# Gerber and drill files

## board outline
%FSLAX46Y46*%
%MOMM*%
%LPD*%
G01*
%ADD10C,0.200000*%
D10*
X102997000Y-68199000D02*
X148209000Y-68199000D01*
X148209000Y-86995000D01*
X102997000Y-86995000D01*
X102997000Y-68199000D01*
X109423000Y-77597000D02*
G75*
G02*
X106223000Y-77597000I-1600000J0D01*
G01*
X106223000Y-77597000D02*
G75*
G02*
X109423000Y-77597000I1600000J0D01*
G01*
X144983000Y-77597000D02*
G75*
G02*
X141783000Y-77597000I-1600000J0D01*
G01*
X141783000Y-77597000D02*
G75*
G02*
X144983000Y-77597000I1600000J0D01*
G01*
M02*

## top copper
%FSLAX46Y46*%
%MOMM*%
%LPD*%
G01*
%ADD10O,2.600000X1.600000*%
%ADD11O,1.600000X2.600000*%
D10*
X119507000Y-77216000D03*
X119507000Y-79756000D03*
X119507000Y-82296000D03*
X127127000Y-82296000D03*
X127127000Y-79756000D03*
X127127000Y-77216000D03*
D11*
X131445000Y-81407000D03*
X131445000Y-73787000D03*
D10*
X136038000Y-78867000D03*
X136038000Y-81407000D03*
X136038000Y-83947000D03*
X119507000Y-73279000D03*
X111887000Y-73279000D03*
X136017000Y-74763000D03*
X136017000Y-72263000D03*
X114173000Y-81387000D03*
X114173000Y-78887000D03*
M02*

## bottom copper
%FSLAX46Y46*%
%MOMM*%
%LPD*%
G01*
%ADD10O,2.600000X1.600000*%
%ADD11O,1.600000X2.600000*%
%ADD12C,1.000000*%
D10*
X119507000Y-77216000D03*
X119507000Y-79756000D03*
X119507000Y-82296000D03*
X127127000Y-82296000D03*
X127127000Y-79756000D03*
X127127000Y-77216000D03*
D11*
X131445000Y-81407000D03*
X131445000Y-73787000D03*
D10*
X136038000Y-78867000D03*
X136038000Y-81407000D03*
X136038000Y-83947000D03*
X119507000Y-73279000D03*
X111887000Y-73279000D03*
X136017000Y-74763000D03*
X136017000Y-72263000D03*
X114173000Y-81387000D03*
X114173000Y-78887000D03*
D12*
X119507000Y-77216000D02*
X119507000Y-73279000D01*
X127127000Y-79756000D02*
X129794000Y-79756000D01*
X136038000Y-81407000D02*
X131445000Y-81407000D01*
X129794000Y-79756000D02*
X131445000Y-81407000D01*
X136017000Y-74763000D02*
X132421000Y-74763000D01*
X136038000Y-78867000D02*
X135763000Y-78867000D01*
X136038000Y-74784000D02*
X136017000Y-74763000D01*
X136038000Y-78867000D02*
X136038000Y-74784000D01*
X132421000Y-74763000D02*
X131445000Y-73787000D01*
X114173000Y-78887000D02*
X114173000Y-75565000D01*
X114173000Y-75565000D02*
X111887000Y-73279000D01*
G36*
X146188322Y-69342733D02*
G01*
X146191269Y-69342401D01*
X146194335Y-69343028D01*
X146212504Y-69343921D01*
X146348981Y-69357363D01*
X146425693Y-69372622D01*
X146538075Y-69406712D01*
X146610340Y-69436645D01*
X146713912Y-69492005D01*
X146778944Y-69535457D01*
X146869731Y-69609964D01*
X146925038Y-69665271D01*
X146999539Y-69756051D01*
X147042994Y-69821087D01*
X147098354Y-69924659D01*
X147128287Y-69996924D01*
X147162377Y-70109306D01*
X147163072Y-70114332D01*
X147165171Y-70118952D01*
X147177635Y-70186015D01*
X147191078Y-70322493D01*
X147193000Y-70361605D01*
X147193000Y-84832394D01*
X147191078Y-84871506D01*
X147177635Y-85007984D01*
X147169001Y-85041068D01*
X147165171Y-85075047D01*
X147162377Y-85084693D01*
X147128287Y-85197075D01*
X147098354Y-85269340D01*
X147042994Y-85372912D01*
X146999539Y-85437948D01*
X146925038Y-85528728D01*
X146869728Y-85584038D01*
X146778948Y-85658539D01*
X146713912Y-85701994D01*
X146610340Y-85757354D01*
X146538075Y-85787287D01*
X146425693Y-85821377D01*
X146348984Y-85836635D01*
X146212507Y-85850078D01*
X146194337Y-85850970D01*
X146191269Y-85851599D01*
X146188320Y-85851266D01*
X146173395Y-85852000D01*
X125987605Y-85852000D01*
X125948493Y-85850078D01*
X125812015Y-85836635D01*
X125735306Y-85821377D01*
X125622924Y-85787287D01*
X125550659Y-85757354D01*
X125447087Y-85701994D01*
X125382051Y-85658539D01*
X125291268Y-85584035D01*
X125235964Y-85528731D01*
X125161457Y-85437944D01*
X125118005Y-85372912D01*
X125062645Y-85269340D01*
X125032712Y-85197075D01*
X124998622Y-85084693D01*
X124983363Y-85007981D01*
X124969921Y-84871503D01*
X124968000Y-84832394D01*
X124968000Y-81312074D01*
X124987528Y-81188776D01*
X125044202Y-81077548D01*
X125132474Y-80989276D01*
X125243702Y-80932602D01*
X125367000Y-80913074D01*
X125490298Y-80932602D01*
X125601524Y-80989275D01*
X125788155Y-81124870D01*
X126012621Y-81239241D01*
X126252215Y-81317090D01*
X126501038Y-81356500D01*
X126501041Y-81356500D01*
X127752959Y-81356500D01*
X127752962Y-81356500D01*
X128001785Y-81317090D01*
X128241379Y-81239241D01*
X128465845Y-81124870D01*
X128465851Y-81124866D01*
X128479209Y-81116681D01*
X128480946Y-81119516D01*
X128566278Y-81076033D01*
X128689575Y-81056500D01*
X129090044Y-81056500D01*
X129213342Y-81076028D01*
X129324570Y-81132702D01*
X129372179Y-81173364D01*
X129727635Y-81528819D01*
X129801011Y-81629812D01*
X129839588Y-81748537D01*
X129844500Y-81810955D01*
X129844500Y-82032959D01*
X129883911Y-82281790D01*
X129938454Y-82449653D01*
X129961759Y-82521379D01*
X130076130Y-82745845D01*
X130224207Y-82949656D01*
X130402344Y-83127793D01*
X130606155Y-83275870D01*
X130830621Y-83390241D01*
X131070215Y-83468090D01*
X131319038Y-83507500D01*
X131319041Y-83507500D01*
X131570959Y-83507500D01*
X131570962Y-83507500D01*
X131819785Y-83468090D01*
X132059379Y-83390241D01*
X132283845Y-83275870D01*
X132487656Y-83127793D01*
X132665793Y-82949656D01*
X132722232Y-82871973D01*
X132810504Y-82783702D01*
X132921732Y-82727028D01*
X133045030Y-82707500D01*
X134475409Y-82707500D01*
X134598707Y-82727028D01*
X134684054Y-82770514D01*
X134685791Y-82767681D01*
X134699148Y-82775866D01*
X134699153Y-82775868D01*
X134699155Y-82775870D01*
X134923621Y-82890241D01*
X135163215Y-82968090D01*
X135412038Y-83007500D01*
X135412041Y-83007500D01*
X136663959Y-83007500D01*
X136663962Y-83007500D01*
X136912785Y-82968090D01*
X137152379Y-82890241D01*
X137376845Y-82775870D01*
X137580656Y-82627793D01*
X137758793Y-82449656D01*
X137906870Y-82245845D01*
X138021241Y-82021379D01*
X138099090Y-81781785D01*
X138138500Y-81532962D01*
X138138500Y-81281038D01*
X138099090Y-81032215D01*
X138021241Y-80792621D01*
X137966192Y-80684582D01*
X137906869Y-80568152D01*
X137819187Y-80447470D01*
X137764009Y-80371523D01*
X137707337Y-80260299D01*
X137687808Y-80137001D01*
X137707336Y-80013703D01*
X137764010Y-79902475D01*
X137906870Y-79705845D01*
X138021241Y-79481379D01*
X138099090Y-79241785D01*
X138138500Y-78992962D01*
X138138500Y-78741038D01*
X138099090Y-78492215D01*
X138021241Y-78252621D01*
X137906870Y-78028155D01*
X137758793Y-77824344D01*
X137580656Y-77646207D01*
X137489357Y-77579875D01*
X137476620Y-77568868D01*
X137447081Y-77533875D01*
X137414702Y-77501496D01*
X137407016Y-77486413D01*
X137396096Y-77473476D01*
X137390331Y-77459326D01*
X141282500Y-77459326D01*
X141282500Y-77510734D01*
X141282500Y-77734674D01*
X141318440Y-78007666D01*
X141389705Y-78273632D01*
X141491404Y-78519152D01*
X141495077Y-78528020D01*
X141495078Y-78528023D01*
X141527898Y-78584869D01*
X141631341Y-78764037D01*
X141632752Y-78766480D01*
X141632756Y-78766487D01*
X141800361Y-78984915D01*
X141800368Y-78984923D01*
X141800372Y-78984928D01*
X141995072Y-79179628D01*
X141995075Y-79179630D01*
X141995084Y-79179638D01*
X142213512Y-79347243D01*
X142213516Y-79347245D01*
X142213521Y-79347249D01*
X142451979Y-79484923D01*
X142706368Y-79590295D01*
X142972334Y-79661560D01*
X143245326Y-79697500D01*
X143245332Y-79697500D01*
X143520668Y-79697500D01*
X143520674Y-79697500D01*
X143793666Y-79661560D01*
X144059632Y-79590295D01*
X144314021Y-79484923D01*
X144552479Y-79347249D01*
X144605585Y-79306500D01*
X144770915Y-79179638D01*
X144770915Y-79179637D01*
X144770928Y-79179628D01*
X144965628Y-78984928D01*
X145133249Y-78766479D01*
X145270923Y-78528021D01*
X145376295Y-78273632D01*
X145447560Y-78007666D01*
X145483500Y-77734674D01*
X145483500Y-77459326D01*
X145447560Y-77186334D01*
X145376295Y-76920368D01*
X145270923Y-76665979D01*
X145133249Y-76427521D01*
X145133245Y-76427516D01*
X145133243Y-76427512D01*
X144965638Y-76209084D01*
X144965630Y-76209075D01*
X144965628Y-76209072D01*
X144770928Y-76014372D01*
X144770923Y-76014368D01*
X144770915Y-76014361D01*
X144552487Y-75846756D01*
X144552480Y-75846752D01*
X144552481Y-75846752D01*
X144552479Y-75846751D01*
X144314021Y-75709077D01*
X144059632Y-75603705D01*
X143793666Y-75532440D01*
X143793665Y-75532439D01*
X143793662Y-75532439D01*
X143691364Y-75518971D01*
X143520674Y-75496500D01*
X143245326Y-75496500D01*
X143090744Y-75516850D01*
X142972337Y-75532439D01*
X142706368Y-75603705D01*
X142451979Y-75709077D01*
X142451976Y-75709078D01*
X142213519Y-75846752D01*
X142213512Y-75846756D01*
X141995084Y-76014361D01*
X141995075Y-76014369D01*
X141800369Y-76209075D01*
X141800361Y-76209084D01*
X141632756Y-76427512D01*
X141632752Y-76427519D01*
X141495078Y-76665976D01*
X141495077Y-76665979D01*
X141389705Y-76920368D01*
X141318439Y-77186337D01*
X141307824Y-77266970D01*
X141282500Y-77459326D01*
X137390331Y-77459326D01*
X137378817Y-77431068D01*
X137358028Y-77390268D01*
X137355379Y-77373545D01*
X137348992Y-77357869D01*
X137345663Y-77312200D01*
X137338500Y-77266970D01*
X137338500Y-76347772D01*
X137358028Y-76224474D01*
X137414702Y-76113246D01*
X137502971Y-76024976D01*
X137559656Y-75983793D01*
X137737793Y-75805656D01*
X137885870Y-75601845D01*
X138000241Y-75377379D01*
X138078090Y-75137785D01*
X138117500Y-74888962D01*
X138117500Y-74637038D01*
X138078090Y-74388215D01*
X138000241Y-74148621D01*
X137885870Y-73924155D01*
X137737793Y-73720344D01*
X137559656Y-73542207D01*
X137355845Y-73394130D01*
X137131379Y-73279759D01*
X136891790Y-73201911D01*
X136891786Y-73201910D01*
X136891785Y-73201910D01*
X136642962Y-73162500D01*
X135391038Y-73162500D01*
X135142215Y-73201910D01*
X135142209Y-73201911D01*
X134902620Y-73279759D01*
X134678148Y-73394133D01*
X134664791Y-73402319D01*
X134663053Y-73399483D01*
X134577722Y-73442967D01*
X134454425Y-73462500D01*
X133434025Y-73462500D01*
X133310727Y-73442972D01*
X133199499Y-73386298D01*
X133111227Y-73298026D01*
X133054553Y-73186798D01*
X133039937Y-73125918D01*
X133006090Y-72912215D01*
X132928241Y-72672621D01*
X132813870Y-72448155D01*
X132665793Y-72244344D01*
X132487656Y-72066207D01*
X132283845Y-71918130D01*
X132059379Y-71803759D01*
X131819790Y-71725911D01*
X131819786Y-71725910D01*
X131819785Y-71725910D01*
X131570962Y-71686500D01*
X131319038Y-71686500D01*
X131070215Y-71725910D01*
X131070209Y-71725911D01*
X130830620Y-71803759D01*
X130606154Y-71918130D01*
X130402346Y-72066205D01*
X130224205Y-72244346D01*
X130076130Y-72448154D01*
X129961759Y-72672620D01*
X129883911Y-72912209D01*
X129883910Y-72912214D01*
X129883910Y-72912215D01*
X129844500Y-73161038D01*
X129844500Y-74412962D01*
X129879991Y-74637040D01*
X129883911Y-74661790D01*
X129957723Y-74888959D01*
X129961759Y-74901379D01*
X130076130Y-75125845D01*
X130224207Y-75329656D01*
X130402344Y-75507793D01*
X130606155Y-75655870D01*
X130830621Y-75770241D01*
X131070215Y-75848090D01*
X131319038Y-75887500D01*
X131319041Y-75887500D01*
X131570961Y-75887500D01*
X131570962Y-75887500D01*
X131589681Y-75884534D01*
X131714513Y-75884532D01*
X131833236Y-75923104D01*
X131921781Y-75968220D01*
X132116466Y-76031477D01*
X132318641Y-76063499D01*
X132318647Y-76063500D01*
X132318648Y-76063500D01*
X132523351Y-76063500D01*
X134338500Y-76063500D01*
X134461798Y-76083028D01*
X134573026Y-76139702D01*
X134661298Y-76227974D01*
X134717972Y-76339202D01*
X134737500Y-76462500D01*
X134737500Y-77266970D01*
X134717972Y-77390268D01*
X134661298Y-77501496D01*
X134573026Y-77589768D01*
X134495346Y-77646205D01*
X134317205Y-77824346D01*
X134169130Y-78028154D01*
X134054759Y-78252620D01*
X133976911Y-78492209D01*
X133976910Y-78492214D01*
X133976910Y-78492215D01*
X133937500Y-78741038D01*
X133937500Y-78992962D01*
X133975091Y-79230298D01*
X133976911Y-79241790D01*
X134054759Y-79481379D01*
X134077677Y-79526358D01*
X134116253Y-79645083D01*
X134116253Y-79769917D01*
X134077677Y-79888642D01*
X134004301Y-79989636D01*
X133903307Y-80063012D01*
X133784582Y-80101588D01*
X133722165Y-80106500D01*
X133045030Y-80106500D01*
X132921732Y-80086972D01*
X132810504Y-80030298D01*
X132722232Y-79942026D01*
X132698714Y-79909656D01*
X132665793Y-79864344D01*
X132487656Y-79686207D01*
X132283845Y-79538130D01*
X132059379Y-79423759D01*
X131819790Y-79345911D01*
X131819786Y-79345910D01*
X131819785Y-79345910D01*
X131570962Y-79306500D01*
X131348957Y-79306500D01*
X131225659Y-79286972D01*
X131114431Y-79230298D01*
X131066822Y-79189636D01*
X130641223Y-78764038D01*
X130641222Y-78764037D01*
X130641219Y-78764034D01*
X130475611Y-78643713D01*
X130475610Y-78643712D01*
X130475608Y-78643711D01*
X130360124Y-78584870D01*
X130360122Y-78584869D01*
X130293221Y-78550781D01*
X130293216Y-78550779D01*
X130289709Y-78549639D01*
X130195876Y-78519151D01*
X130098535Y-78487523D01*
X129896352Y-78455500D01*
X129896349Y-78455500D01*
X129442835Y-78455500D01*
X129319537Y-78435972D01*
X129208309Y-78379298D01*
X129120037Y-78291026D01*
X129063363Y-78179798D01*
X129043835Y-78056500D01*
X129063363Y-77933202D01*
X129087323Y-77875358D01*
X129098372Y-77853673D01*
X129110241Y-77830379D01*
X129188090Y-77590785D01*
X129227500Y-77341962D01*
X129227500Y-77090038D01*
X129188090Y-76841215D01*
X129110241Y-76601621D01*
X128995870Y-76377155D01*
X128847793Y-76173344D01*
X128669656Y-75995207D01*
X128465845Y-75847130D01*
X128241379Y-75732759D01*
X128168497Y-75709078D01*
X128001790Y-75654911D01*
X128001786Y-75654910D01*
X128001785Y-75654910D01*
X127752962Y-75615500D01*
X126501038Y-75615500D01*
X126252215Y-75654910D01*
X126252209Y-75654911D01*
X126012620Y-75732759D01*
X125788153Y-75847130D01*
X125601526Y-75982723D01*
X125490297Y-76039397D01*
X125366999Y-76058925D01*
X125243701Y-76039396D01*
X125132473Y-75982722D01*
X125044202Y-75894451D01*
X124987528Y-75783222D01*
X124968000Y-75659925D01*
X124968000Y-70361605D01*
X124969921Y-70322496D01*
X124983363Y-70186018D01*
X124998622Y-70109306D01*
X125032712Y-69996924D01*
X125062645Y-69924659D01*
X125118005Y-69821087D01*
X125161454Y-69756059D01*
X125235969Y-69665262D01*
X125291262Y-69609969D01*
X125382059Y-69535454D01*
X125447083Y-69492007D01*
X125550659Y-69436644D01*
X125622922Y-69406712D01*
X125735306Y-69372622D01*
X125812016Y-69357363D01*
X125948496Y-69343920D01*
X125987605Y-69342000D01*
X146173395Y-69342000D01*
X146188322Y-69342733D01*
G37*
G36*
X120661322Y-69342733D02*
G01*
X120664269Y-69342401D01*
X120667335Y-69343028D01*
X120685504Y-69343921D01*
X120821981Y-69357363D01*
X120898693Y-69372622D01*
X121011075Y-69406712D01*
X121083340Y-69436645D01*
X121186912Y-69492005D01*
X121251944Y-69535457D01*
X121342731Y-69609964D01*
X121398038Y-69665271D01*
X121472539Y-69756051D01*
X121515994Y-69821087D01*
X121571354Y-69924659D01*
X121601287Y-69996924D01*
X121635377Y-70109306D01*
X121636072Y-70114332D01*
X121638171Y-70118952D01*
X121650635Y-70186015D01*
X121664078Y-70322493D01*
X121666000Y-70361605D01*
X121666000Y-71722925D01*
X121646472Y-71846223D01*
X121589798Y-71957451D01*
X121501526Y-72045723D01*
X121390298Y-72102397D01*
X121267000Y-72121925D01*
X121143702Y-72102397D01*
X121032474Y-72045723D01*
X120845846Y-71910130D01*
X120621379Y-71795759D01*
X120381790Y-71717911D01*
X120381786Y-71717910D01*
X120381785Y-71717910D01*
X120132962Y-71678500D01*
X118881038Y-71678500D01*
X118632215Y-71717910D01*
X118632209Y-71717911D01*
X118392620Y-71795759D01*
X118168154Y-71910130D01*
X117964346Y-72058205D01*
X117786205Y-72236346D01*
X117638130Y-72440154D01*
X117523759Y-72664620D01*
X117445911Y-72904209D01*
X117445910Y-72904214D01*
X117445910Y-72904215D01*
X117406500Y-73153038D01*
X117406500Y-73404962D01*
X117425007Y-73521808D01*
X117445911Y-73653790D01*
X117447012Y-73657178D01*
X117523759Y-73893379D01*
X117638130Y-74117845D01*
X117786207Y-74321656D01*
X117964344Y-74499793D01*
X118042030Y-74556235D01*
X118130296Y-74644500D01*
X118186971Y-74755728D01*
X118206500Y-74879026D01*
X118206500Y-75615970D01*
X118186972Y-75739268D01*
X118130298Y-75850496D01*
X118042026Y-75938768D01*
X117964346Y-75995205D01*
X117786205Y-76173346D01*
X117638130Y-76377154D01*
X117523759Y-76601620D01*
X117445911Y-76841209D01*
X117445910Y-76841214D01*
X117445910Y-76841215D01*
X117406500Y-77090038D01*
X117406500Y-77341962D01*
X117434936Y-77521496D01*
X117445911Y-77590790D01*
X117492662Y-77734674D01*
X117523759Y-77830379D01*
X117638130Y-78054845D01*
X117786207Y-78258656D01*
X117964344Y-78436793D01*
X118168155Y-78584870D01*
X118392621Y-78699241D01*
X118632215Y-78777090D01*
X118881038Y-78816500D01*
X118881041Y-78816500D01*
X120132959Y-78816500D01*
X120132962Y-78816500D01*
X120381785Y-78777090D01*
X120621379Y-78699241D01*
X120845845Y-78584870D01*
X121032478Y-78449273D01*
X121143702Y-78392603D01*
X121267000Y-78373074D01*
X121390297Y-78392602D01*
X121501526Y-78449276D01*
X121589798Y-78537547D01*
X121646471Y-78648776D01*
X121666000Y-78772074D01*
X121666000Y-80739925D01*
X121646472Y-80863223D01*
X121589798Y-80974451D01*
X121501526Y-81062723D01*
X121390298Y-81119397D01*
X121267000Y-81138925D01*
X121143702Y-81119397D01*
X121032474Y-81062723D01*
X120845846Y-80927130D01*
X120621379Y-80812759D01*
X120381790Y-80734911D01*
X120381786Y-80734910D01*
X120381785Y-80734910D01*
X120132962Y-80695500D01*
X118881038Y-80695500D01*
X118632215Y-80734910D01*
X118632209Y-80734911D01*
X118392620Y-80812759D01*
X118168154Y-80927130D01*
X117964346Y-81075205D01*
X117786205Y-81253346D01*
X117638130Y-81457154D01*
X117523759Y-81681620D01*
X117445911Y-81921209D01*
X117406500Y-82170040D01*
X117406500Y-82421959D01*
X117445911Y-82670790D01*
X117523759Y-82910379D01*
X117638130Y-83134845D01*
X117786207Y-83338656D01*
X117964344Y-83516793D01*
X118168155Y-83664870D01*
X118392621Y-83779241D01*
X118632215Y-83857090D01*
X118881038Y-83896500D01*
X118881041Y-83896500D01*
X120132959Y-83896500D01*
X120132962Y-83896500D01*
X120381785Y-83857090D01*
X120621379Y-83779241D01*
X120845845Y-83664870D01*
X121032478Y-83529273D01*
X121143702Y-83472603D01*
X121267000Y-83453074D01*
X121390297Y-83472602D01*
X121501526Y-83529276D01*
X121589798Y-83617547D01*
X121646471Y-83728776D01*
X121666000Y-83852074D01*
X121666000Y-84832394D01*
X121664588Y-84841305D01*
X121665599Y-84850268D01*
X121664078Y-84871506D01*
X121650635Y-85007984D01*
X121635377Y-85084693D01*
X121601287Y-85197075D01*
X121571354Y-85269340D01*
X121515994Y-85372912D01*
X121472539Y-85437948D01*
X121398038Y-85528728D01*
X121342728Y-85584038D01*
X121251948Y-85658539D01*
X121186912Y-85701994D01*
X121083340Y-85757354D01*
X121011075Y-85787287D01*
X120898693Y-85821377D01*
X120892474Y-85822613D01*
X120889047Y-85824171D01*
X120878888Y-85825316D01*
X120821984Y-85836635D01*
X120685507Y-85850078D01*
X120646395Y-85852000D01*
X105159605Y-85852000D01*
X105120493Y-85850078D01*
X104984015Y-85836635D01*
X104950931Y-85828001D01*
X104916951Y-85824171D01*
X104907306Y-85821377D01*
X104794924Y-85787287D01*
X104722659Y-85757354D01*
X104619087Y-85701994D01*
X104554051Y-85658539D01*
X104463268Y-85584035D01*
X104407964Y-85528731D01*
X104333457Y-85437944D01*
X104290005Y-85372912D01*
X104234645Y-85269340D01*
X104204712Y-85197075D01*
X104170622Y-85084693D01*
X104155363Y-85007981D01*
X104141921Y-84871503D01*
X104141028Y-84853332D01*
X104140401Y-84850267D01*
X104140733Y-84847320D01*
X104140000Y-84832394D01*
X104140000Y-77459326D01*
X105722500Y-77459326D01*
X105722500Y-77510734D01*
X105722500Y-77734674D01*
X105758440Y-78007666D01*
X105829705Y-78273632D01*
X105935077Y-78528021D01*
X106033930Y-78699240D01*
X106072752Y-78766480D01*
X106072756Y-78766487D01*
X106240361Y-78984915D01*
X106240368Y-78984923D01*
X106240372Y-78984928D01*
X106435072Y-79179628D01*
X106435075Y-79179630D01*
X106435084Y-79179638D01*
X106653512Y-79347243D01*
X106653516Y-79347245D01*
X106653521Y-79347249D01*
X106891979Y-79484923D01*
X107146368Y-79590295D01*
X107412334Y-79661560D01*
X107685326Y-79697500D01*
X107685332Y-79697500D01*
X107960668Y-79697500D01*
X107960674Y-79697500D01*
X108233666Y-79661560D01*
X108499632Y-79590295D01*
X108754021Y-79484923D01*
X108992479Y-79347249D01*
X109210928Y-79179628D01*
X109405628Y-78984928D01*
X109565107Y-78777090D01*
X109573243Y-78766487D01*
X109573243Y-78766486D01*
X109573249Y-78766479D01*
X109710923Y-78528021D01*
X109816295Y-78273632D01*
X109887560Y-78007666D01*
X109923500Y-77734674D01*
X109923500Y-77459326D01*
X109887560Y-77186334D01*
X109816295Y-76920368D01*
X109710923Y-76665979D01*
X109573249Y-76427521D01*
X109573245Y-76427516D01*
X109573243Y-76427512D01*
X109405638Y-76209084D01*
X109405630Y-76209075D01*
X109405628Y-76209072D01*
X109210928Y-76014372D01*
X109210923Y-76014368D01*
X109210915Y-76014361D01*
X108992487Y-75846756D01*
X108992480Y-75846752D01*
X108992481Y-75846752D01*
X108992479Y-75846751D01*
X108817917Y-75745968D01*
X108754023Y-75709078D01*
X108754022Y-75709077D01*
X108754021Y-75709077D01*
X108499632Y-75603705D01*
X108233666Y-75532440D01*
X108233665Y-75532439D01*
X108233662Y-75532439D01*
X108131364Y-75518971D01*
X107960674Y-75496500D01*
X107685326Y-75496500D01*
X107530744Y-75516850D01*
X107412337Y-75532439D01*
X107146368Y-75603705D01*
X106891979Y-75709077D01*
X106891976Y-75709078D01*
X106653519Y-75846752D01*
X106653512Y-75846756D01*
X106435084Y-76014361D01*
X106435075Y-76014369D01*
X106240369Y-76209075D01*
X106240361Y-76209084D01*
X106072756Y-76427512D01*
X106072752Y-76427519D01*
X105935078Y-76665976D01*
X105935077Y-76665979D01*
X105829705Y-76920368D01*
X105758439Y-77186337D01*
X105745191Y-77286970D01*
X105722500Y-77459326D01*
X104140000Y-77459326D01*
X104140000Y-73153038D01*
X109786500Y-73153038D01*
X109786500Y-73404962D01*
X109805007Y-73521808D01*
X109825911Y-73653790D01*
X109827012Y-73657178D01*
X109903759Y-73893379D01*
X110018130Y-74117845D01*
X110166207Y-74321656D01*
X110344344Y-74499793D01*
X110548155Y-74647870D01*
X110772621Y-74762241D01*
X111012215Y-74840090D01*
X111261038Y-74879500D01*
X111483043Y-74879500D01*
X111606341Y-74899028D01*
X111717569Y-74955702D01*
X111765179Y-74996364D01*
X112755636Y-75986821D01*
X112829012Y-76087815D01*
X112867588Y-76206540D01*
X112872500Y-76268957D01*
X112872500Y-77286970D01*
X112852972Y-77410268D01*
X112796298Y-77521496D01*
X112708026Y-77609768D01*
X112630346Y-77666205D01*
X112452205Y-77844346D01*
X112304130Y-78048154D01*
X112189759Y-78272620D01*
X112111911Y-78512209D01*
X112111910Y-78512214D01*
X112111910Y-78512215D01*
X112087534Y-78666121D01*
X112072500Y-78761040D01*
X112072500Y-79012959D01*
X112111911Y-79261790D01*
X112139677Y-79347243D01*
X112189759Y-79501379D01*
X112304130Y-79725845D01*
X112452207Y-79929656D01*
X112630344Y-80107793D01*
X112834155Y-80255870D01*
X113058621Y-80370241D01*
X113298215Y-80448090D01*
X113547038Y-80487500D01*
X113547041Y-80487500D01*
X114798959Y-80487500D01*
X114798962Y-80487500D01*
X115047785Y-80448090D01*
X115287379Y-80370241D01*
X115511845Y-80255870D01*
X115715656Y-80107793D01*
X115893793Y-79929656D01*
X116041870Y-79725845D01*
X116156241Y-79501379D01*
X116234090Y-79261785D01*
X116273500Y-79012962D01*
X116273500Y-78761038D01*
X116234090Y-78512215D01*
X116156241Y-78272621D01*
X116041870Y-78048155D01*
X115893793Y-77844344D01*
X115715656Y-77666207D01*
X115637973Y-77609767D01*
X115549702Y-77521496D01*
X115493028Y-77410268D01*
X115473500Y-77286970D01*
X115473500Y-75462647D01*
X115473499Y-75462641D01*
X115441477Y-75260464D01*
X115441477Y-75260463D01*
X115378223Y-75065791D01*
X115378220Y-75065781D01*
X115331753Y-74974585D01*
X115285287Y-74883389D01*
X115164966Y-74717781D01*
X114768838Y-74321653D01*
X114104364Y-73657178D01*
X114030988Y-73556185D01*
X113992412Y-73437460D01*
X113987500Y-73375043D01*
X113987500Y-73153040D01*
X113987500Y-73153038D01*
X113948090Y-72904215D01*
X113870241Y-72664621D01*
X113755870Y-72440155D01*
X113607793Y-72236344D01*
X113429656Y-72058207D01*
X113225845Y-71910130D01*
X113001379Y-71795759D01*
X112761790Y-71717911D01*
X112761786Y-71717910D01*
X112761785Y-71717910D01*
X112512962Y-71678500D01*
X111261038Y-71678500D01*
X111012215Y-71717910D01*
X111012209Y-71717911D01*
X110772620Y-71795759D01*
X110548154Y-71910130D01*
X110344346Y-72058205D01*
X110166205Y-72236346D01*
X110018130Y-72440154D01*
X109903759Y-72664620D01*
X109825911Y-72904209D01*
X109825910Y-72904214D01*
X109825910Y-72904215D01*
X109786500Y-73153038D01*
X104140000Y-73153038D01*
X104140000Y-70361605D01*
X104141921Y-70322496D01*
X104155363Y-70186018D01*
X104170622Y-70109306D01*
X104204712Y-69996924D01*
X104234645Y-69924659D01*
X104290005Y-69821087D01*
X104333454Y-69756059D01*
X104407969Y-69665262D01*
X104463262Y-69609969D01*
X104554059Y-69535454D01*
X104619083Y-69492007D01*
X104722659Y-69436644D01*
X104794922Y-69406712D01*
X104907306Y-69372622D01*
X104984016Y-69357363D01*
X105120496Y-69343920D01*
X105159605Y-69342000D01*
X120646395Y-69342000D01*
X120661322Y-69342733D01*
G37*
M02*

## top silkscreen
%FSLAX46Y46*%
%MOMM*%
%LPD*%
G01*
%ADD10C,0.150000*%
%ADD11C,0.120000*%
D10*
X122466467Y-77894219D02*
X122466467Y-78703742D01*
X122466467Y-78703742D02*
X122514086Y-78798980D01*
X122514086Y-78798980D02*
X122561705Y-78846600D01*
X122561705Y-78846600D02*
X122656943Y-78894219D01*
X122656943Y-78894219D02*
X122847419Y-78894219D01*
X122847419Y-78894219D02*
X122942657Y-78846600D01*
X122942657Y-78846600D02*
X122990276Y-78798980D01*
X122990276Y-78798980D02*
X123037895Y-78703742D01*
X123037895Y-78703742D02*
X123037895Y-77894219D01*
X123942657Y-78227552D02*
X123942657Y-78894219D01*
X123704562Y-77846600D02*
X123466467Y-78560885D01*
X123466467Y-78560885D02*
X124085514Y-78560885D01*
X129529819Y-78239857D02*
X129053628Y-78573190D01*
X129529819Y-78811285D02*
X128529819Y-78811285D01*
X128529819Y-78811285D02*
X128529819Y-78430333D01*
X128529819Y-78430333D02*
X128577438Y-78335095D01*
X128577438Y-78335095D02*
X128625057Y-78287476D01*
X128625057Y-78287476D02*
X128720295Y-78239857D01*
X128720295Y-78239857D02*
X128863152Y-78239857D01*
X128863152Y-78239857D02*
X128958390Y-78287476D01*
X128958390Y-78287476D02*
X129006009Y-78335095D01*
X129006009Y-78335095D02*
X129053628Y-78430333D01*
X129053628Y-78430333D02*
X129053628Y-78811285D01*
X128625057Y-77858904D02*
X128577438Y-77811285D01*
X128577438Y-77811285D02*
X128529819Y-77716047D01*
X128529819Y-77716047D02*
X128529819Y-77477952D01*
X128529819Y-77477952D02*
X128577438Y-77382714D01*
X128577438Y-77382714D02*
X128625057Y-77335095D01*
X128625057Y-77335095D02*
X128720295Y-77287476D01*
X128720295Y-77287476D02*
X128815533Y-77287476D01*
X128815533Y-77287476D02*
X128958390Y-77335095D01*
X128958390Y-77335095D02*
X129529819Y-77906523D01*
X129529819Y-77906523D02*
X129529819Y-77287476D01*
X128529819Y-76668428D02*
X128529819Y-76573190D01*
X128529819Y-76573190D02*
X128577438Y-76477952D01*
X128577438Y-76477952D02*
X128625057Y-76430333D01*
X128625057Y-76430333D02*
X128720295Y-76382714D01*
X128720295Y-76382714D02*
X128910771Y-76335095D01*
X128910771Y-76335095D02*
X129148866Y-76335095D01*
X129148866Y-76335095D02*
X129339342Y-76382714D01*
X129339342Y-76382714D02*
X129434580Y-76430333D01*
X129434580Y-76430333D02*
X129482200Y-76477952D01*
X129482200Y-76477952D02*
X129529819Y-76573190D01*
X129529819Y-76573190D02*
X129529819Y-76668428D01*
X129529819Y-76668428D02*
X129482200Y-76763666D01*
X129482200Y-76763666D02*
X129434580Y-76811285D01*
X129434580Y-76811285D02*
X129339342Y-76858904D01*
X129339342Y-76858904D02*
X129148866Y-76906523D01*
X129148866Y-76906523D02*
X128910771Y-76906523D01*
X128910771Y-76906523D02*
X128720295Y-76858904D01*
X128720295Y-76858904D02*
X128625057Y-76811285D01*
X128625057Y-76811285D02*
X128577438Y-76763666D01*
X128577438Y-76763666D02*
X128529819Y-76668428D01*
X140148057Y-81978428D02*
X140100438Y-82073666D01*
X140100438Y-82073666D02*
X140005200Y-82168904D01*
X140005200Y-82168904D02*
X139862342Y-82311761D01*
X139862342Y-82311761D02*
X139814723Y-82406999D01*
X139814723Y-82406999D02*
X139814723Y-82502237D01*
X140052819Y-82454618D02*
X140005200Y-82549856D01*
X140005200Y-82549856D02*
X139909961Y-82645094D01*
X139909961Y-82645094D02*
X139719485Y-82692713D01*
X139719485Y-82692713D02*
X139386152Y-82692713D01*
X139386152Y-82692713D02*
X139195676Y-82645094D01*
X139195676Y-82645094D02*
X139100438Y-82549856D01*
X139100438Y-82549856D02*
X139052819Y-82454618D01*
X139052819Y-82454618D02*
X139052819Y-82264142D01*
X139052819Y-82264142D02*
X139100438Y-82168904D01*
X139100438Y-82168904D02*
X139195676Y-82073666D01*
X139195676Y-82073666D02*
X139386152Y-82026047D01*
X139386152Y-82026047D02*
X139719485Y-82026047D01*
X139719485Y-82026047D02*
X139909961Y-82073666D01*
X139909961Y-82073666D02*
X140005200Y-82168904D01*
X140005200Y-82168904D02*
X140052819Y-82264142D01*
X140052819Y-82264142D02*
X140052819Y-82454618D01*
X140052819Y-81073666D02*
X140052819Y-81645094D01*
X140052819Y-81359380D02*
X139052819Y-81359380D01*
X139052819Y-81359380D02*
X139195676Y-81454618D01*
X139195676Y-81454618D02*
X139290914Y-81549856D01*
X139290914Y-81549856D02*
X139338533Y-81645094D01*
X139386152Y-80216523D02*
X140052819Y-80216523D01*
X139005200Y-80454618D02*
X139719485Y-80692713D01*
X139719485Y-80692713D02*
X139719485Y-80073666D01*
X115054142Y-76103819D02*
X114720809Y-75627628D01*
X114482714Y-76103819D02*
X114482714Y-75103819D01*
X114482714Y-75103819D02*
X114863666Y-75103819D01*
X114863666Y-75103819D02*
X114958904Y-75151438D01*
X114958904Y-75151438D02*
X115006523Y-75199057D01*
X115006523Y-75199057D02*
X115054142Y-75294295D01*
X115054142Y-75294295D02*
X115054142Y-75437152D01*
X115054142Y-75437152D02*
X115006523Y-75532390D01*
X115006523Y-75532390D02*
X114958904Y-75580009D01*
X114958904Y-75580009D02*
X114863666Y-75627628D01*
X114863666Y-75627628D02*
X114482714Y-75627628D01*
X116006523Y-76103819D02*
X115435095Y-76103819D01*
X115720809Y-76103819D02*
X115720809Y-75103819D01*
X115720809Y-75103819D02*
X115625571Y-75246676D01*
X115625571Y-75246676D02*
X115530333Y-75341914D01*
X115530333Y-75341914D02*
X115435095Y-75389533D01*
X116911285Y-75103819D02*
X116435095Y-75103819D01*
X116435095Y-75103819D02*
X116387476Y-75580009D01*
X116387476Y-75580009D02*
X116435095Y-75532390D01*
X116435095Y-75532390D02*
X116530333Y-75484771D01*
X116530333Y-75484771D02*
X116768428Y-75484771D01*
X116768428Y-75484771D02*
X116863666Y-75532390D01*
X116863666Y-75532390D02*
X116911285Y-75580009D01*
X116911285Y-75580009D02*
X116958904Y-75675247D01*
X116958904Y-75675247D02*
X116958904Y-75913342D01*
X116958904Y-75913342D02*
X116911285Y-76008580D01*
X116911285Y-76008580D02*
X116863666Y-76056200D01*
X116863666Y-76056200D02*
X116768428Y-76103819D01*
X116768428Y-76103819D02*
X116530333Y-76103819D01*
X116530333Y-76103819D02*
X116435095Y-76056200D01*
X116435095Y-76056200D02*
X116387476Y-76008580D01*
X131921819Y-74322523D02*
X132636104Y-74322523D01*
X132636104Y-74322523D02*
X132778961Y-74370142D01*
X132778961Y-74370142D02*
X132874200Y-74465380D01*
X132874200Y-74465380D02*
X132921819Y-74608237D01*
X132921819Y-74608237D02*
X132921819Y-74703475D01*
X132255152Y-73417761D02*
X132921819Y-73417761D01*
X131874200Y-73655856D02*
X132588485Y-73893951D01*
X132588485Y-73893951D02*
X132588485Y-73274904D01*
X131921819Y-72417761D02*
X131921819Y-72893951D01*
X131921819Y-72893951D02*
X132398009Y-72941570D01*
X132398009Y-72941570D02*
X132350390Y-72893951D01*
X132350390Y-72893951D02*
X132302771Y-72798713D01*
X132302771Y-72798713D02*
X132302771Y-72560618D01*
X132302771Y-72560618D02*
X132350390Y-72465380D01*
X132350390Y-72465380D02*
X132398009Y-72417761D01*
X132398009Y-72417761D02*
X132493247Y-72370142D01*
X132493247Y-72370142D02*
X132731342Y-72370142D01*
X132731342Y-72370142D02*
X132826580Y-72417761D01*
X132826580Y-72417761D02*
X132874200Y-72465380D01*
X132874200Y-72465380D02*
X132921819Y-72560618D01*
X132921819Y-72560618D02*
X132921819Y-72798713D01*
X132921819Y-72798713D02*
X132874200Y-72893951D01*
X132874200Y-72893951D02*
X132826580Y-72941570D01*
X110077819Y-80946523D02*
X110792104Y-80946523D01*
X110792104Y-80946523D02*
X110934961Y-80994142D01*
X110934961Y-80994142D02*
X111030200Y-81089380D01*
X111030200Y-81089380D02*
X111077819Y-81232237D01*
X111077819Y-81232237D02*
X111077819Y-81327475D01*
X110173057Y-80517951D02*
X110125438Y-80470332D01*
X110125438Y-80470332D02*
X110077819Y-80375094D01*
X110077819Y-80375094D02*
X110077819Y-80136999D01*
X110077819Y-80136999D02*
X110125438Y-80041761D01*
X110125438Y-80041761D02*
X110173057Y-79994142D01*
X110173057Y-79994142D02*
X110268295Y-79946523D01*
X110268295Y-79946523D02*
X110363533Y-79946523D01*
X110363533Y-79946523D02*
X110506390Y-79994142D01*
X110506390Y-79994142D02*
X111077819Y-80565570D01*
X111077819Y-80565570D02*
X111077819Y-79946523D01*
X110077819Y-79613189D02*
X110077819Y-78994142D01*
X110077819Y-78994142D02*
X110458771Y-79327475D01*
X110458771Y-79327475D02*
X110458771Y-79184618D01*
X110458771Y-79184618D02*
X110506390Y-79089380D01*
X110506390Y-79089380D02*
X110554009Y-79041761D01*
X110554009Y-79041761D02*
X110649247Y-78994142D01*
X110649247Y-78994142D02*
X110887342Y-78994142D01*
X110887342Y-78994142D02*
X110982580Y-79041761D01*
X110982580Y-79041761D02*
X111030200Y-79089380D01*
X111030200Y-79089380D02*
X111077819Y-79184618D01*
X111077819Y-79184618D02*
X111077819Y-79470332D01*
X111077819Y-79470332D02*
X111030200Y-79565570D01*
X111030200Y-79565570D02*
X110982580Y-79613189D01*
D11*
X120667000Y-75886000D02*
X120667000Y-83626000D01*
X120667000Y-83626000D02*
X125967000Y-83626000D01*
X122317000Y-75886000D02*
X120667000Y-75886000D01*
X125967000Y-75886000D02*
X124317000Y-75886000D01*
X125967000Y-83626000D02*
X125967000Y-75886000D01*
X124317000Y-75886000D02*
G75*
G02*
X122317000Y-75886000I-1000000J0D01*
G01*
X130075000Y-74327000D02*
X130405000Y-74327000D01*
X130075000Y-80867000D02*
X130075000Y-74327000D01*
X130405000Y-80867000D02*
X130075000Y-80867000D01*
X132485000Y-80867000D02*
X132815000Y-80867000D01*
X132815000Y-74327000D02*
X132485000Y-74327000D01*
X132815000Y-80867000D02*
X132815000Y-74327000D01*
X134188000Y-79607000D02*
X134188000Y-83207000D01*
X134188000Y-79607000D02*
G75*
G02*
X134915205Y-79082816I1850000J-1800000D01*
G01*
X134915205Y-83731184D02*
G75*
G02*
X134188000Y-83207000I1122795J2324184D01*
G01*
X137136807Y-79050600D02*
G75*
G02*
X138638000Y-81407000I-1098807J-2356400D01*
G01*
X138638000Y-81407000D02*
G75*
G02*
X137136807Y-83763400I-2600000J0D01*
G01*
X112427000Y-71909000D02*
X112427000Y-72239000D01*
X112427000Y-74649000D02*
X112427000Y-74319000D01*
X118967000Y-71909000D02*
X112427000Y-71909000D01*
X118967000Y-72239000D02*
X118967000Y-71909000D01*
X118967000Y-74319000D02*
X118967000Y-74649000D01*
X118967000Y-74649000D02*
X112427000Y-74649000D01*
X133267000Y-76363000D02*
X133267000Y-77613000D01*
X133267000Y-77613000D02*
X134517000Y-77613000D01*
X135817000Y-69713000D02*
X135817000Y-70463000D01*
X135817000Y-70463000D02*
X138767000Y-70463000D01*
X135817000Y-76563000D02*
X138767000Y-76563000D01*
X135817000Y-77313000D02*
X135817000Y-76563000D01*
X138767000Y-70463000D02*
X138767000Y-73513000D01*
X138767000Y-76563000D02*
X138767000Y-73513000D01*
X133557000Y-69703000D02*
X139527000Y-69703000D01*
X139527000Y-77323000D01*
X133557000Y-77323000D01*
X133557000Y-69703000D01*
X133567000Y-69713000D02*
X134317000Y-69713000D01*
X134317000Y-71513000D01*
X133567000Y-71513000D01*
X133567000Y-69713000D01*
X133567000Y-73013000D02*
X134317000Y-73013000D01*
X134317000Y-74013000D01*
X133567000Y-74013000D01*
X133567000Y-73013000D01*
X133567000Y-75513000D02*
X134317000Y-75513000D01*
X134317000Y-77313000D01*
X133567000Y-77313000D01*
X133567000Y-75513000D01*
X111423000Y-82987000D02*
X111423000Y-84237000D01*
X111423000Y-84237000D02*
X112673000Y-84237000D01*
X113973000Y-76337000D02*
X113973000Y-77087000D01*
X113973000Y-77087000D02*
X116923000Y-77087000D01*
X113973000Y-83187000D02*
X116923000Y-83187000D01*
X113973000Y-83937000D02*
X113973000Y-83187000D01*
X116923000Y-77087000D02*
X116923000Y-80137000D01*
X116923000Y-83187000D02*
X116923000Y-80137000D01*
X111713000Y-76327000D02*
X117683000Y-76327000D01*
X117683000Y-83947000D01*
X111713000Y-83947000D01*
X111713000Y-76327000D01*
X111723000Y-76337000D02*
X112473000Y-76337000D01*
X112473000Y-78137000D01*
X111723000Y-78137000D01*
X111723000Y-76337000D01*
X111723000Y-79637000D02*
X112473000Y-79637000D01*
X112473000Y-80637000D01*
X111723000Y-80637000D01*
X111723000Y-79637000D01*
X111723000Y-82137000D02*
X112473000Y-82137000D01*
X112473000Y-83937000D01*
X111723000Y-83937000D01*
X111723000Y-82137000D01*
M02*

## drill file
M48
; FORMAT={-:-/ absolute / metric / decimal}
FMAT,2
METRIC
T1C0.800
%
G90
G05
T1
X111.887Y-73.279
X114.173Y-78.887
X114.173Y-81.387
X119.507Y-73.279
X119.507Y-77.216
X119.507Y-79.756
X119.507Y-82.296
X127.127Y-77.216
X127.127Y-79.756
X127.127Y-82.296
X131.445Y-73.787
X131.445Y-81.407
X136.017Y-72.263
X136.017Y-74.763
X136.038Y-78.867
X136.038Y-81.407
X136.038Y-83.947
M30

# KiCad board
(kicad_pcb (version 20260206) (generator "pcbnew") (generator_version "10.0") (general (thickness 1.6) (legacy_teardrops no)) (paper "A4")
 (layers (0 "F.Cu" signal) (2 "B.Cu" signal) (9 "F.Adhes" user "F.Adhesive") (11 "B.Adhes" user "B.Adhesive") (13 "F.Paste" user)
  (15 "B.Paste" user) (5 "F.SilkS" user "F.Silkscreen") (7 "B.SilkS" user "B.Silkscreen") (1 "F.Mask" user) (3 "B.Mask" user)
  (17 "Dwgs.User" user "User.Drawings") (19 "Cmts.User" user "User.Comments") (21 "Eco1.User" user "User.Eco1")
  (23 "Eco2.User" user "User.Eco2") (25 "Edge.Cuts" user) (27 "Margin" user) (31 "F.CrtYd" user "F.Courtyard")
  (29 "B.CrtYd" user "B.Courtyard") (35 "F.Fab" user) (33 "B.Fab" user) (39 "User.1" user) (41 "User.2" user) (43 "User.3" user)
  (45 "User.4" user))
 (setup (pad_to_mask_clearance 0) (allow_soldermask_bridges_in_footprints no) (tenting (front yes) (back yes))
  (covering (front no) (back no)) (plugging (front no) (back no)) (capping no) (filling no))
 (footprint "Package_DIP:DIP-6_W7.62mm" (layer "F.Cu") (at 119.507 77.216)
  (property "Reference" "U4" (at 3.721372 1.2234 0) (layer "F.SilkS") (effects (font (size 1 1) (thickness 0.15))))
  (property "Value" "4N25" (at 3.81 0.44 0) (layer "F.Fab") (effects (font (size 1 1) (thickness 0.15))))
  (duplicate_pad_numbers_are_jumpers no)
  (fp_line (start 1.16 -1.33) (end 1.16 6.41) (stroke (width 0.12) (type solid)) (layer "F.SilkS"))
  (fp_line (start 1.16 6.41) (end 6.46 6.41) (stroke (width 0.12) (type solid)) (layer "F.SilkS"))
  (fp_line (start 2.81 -1.33) (end 1.16 -1.33) (stroke (width 0.12) (type solid)) (layer "F.SilkS"))
  (fp_line (start 6.46 -1.33) (end 4.81 -1.33) (stroke (width 0.12) (type solid)) (layer "F.SilkS"))
  (fp_line (start 6.46 6.41) (end 6.46 -1.33) (stroke (width 0.12) (type solid)) (layer "F.SilkS"))
  (fp_arc (start 4.81 -1.33) (mid 3.81 -0.33) (end 2.81 -1.33) (stroke (width 0.12) (type solid)) (layer "F.SilkS"))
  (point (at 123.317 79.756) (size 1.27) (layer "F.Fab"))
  (pad "1" thru_hole oval (at 0 0 90) (size 1.6 2.6) (drill 0.8) (layers "*.Cu" "*.Mask") (remove_unused_layers no) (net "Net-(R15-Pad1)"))
  (pad "2" thru_hole oval (at 0 2.54 90) (size 1.6 2.6) (drill 0.8) (layers "*.Cu" "*.Mask") (remove_unused_layers no) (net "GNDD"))
  (pad "3" thru_hole oval (at 0 5.08 90) (size 1.6 2.6) (drill 0.8) (layers "*.Cu" "*.Mask") (remove_unused_layers no)
   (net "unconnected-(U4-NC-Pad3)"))
  (pad "4" thru_hole oval (at 7.62 5.08 90) (size 1.6 2.6) (drill 0.8) (layers "*.Cu" "*.Mask") (remove_unused_layers no)
   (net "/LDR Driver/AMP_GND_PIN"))
  (pad "5" thru_hole oval (at 7.62 2.54 90) (size 1.6 2.6) (drill 0.8) (layers "*.Cu" "*.Mask") (remove_unused_layers no)
   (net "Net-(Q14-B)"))
  (pad "6" thru_hole oval (at 7.62 0 90) (size 1.6 2.6) (drill 0.8) (layers "*.Cu" "*.Mask") (remove_unused_layers no)
   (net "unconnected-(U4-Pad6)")))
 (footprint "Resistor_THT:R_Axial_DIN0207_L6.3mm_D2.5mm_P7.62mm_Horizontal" (layer "F.Cu") (at 131.445 81.407 90)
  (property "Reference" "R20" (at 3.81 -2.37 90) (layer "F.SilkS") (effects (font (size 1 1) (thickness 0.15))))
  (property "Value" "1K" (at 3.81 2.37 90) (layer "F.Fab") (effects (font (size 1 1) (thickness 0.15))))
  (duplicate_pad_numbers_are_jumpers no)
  (fp_line (start 7.08 -1.37) (end 7.08 -1.04) (stroke (width 0.12) (type solid)) (layer "F.SilkS"))
  (fp_line (start 0.54 -1.37) (end 7.08 -1.37) (stroke (width 0.12) (type solid)) (layer "F.SilkS"))
  (fp_line (start 0.54 -1.04) (end 0.54 -1.37) (stroke (width 0.12) (type solid)) (layer "F.SilkS"))
  (fp_line (start 0.54 1.04) (end 0.54 1.37) (stroke (width 0.12) (type solid)) (layer "F.SilkS"))
  (fp_line (start 7.08 1.37) (end 7.08 1.04) (stroke (width 0.12) (type solid)) (layer "F.SilkS"))
  (fp_line (start 0.54 1.37) (end 7.08 1.37) (stroke (width 0.12) (type solid)) (layer "F.SilkS"))
  (pad "1" thru_hole oval (at 0 0 180) (size 1.6 2.6) (drill 0.8) (layers "*.Cu" "*.Mask") (remove_unused_layers no) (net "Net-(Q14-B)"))
  (pad "2" thru_hole oval (at 7.62 0 180) (size 1.6 2.6) (drill 0.8) (layers "*.Cu" "*.Mask") (remove_unused_layers no)
   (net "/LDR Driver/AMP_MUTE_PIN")))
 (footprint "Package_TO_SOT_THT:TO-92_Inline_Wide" (layer "F.Cu") (at 136.038 78.867 -90)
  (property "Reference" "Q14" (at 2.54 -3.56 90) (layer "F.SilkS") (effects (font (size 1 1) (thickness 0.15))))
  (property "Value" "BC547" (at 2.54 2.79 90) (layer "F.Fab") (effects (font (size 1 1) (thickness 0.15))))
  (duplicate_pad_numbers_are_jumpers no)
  (fp_line (start 0.74 1.85) (end 4.34 1.85) (stroke (width 0.12) (type solid)) (layer "F.SilkS"))
  (fp_arc (start 0.74 1.85) (mid 0.446097 1.509328) (end 0.215816 1.122795) (stroke (width 0.12) (type solid)) (layer "F.SilkS"))
  (fp_arc (start 4.864184 1.122795) (mid 4.633903 1.509328) (end 4.34 1.85) (stroke (width 0.12) (type solid)) (layer "F.SilkS"))
  (fp_arc (start 0.1836 -1.098807) (mid 1.143021 -2.192817) (end 2.54 -2.6) (stroke (width 0.12) (type solid)) (layer "F.SilkS"))
  (fp_arc (start 2.54 -2.6) (mid 3.936979 -2.192818) (end 4.8964 -1.098807) (stroke (width 0.12) (type solid)) (layer "F.SilkS"))
  (pad "1" thru_hole oval (at 0 0 270) (size 1.6 2.6) (drill 0.8) (layers "*.Cu" "*.Mask") (remove_unused_layers no)
   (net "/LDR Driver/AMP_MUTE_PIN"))
  (pad "2" thru_hole oval (at 2.54 0 270) (size 1.6 2.6) (drill 0.8) (layers "*.Cu" "*.Mask") (remove_unused_layers no) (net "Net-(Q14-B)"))
  (pad "3" thru_hole oval (at 5.08 0 270) (size 1.6 2.6) (drill 0.8) (layers "*.Cu" "*.Mask") (remove_unused_layers no)
   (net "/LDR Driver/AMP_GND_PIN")))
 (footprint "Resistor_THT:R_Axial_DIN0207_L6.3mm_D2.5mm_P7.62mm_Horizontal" (layer "F.Cu") (at 119.507 73.279 180)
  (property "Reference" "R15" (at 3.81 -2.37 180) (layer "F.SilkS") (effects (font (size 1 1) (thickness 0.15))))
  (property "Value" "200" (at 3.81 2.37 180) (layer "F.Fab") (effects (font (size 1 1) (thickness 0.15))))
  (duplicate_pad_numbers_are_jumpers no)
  (fp_line (start 7.08 1.37) (end 7.08 1.04) (stroke (width 0.12) (type solid)) (layer "F.SilkS"))
  (fp_line (start 7.08 -1.37) (end 7.08 -1.04) (stroke (width 0.12) (type solid)) (layer "F.SilkS"))
  (fp_line (start 0.54 1.37) (end 7.08 1.37) (stroke (width 0.12) (type solid)) (layer "F.SilkS"))
  (fp_line (start 0.54 1.04) (end 0.54 1.37) (stroke (width 0.12) (type solid)) (layer "F.SilkS"))
  (fp_line (start 0.54 -1.04) (end 0.54 -1.37) (stroke (width 0.12) (type solid)) (layer "F.SilkS"))
  (fp_line (start 0.54 -1.37) (end 7.08 -1.37) (stroke (width 0.12) (type solid)) (layer "F.SilkS"))
  (pad "1" thru_hole oval (at 0 0 270) (size 1.6 2.6) (drill 0.8) (layers "*.Cu" "*.Mask") (remove_unused_layers no) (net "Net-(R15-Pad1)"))
  (pad "2" thru_hole oval (at 7.62 0 270) (size 1.6 2.6) (drill 0.8) (layers "*.Cu" "*.Mask") (remove_unused_layers no)
   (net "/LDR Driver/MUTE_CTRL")))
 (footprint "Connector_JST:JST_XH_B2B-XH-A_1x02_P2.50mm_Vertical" (layer "F.Cu") (at 136.017 74.763 90)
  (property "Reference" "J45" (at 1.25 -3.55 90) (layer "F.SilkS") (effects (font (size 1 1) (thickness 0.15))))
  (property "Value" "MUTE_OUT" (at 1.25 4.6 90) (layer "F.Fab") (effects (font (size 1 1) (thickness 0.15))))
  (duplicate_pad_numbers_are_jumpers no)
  (fp_line (start -1.6 -2.75) (end -2.85 -2.75) (stroke (width 0.12) (type solid)) (layer "F.SilkS"))
  (fp_line (start -2.85 -2.75) (end -2.85 -1.5) (stroke (width 0.12) (type solid)) (layer "F.SilkS"))
  (fp_line (start 5.05 -0.2) (end 4.3 -0.2) (stroke (width 0.12) (type solid)) (layer "F.SilkS"))
  (fp_line (start 4.3 -0.2) (end 4.3 2.75) (stroke (width 0.12) (type solid)) (layer "F.SilkS"))
  (fp_line (start -1.8 -0.2) (end -1.8 2.75) (stroke (width 0.12) (type solid)) (layer "F.SilkS"))
  (fp_line (start -2.55 -0.2) (end -1.8 -0.2) (stroke (width 0.12) (type solid)) (layer "F.SilkS"))
  (fp_line (start 4.3 2.75) (end 1.25 2.75) (stroke (width 0.12) (type solid)) (layer "F.SilkS"))
  (fp_line (start -1.8 2.75) (end 1.25 2.75) (stroke (width 0.12) (type solid)) (layer "F.SilkS"))
  (fp_rect (start -2.56 -2.46) (end 5.06 3.51) (stroke (width 0.12) (type solid)) (fill no) (layer "F.SilkS"))
  (fp_rect (start 3.25 -2.45) (end 5.05 -1.7) (stroke (width 0.12) (type solid)) (fill no) (layer "F.SilkS"))
  (fp_rect (start 0.75 -2.45) (end 1.75 -1.7) (stroke (width 0.12) (type solid)) (fill no) (layer "F.SilkS"))
  (fp_rect (start -2.55 -2.45) (end -0.75 -1.7) (stroke (width 0.12) (type solid)) (fill no) (layer "F.SilkS"))
  (pad "1" thru_hole oval (at 0 0 90) (size 1.6 2.6) (drill 0.8) (layers "*.Cu" "*.Mask") (remove_unused_layers no)
   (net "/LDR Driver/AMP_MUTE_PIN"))
  (pad "2" thru_hole oval (at 2.5 0 90) (size 1.6 2.6) (drill 0.8) (layers "*.Cu" "*.Mask") (remove_unused_layers no)
   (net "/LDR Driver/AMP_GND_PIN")))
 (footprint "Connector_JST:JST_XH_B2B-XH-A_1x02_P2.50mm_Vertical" (layer "F.Cu") (at 114.173 81.387 90)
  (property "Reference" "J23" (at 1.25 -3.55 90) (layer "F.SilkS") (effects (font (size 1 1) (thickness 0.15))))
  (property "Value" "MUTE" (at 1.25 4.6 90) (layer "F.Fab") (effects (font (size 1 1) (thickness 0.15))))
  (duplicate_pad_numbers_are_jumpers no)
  (fp_line (start -1.6 -2.75) (end -2.85 -2.75) (stroke (width 0.12) (type solid)) (layer "F.SilkS"))
  (fp_line (start -2.85 -2.75) (end -2.85 -1.5) (stroke (width 0.12) (type solid)) (layer "F.SilkS"))
  (fp_line (start 5.05 -0.2) (end 4.3 -0.2) (stroke (width 0.12) (type solid)) (layer "F.SilkS"))
  (fp_line (start 4.3 -0.2) (end 4.3 2.75) (stroke (width 0.12) (type solid)) (layer "F.SilkS"))
  (fp_line (start -1.8 -0.2) (end -1.8 2.75) (stroke (width 0.12) (type solid)) (layer "F.SilkS"))
  (fp_line (start -2.55 -0.2) (end -1.8 -0.2) (stroke (width 0.12) (type solid)) (layer "F.SilkS"))
  (fp_line (start 4.3 2.75) (end 1.25 2.75) (stroke (width 0.12) (type solid)) (layer "F.SilkS"))
  (fp_line (start -1.8 2.75) (end 1.25 2.75) (stroke (width 0.12) (type solid)) (layer "F.SilkS"))
  (fp_rect (start -2.56 -2.46) (end 5.06 3.51) (stroke (width 0.12) (type solid)) (fill no) (layer "F.SilkS"))
  (fp_rect (start 3.25 -2.45) (end 5.05 -1.7) (stroke (width 0.12) (type solid)) (fill no) (layer "F.SilkS"))
  (fp_rect (start 0.75 -2.45) (end 1.75 -1.7) (stroke (width 0.12) (type solid)) (fill no) (layer "F.SilkS"))
  (fp_rect (start -2.55 -2.45) (end -0.75 -1.7) (stroke (width 0.12) (type solid)) (fill no) (layer "F.SilkS"))
  (pad "1" thru_hole oval (at 0 0 90) (size 1.6 2.6) (drill 0.8) (layers "*.Cu" "*.Mask") (remove_unused_layers no) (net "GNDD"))
  (pad "2" thru_hole oval (at 2.5 0 90) (size 1.6 2.6) (drill 0.8) (layers "*.Cu" "*.Mask") (remove_unused_layers no)
   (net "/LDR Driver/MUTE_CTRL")))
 (gr_rect (start 102.997 68.199) (end 148.209 86.995) (stroke (width 0.2) (type solid)) (fill no) (layer "Edge.Cuts"))
 (gr_circle (center 107.823 77.597) (end 109.423 77.597) (stroke (width 0.2) (type solid)) (fill no) (layer "Edge.Cuts"))
 (gr_circle (center 143.383 77.597) (end 144.983 77.597) (stroke (width 0.2) (type solid)) (fill no) (layer "Edge.Cuts"))
 (segment (start 119.507 77.216) (end 119.507 73.279) (width 1) (layer "B.Cu") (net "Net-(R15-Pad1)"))
 (segment (start 127.127 79.756) (end 129.794 79.756) (width 1) (layer "B.Cu") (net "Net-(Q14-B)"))
 (segment (start 136.038 81.407) (end 131.445 81.407) (width 1) (layer "B.Cu") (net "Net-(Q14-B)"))
 (segment (start 129.794 79.756) (end 131.445 81.407) (width 1) (layer "B.Cu") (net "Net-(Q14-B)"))
 (segment (start 136.017 74.763) (end 132.421 74.763) (width 1) (layer "B.Cu") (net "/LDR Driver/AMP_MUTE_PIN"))
 (segment (start 136.038 78.867) (end 135.763 78.867) (width 1) (layer "B.Cu") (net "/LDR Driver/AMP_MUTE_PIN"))
 (segment (start 136.038 74.784) (end 136.017 74.763) (width 1) (layer "B.Cu") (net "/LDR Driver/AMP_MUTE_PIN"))
 (segment (start 136.038 78.867) (end 136.038 74.784) (width 1) (layer "B.Cu") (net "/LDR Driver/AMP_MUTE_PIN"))
 (segment (start 132.421 74.763) (end 131.445 73.787) (width 1) (layer "B.Cu") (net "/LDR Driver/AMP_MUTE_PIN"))
 (segment (start 114.173 78.887) (end 114.173 75.565) (width 1) (layer "B.Cu") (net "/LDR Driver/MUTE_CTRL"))
 (segment (start 114.173 75.565) (end 111.887 73.279) (width 1) (layer "B.Cu") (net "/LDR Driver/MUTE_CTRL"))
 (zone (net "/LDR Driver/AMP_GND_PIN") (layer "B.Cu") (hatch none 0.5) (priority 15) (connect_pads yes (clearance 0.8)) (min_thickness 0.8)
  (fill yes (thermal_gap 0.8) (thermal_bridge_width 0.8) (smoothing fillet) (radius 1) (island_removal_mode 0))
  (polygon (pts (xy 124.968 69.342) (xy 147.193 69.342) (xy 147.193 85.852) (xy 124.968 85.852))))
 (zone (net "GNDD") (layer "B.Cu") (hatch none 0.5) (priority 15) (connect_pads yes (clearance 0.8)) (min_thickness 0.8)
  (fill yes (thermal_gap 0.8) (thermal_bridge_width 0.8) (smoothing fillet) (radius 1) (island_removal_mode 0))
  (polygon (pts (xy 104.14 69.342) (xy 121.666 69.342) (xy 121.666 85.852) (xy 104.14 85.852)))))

